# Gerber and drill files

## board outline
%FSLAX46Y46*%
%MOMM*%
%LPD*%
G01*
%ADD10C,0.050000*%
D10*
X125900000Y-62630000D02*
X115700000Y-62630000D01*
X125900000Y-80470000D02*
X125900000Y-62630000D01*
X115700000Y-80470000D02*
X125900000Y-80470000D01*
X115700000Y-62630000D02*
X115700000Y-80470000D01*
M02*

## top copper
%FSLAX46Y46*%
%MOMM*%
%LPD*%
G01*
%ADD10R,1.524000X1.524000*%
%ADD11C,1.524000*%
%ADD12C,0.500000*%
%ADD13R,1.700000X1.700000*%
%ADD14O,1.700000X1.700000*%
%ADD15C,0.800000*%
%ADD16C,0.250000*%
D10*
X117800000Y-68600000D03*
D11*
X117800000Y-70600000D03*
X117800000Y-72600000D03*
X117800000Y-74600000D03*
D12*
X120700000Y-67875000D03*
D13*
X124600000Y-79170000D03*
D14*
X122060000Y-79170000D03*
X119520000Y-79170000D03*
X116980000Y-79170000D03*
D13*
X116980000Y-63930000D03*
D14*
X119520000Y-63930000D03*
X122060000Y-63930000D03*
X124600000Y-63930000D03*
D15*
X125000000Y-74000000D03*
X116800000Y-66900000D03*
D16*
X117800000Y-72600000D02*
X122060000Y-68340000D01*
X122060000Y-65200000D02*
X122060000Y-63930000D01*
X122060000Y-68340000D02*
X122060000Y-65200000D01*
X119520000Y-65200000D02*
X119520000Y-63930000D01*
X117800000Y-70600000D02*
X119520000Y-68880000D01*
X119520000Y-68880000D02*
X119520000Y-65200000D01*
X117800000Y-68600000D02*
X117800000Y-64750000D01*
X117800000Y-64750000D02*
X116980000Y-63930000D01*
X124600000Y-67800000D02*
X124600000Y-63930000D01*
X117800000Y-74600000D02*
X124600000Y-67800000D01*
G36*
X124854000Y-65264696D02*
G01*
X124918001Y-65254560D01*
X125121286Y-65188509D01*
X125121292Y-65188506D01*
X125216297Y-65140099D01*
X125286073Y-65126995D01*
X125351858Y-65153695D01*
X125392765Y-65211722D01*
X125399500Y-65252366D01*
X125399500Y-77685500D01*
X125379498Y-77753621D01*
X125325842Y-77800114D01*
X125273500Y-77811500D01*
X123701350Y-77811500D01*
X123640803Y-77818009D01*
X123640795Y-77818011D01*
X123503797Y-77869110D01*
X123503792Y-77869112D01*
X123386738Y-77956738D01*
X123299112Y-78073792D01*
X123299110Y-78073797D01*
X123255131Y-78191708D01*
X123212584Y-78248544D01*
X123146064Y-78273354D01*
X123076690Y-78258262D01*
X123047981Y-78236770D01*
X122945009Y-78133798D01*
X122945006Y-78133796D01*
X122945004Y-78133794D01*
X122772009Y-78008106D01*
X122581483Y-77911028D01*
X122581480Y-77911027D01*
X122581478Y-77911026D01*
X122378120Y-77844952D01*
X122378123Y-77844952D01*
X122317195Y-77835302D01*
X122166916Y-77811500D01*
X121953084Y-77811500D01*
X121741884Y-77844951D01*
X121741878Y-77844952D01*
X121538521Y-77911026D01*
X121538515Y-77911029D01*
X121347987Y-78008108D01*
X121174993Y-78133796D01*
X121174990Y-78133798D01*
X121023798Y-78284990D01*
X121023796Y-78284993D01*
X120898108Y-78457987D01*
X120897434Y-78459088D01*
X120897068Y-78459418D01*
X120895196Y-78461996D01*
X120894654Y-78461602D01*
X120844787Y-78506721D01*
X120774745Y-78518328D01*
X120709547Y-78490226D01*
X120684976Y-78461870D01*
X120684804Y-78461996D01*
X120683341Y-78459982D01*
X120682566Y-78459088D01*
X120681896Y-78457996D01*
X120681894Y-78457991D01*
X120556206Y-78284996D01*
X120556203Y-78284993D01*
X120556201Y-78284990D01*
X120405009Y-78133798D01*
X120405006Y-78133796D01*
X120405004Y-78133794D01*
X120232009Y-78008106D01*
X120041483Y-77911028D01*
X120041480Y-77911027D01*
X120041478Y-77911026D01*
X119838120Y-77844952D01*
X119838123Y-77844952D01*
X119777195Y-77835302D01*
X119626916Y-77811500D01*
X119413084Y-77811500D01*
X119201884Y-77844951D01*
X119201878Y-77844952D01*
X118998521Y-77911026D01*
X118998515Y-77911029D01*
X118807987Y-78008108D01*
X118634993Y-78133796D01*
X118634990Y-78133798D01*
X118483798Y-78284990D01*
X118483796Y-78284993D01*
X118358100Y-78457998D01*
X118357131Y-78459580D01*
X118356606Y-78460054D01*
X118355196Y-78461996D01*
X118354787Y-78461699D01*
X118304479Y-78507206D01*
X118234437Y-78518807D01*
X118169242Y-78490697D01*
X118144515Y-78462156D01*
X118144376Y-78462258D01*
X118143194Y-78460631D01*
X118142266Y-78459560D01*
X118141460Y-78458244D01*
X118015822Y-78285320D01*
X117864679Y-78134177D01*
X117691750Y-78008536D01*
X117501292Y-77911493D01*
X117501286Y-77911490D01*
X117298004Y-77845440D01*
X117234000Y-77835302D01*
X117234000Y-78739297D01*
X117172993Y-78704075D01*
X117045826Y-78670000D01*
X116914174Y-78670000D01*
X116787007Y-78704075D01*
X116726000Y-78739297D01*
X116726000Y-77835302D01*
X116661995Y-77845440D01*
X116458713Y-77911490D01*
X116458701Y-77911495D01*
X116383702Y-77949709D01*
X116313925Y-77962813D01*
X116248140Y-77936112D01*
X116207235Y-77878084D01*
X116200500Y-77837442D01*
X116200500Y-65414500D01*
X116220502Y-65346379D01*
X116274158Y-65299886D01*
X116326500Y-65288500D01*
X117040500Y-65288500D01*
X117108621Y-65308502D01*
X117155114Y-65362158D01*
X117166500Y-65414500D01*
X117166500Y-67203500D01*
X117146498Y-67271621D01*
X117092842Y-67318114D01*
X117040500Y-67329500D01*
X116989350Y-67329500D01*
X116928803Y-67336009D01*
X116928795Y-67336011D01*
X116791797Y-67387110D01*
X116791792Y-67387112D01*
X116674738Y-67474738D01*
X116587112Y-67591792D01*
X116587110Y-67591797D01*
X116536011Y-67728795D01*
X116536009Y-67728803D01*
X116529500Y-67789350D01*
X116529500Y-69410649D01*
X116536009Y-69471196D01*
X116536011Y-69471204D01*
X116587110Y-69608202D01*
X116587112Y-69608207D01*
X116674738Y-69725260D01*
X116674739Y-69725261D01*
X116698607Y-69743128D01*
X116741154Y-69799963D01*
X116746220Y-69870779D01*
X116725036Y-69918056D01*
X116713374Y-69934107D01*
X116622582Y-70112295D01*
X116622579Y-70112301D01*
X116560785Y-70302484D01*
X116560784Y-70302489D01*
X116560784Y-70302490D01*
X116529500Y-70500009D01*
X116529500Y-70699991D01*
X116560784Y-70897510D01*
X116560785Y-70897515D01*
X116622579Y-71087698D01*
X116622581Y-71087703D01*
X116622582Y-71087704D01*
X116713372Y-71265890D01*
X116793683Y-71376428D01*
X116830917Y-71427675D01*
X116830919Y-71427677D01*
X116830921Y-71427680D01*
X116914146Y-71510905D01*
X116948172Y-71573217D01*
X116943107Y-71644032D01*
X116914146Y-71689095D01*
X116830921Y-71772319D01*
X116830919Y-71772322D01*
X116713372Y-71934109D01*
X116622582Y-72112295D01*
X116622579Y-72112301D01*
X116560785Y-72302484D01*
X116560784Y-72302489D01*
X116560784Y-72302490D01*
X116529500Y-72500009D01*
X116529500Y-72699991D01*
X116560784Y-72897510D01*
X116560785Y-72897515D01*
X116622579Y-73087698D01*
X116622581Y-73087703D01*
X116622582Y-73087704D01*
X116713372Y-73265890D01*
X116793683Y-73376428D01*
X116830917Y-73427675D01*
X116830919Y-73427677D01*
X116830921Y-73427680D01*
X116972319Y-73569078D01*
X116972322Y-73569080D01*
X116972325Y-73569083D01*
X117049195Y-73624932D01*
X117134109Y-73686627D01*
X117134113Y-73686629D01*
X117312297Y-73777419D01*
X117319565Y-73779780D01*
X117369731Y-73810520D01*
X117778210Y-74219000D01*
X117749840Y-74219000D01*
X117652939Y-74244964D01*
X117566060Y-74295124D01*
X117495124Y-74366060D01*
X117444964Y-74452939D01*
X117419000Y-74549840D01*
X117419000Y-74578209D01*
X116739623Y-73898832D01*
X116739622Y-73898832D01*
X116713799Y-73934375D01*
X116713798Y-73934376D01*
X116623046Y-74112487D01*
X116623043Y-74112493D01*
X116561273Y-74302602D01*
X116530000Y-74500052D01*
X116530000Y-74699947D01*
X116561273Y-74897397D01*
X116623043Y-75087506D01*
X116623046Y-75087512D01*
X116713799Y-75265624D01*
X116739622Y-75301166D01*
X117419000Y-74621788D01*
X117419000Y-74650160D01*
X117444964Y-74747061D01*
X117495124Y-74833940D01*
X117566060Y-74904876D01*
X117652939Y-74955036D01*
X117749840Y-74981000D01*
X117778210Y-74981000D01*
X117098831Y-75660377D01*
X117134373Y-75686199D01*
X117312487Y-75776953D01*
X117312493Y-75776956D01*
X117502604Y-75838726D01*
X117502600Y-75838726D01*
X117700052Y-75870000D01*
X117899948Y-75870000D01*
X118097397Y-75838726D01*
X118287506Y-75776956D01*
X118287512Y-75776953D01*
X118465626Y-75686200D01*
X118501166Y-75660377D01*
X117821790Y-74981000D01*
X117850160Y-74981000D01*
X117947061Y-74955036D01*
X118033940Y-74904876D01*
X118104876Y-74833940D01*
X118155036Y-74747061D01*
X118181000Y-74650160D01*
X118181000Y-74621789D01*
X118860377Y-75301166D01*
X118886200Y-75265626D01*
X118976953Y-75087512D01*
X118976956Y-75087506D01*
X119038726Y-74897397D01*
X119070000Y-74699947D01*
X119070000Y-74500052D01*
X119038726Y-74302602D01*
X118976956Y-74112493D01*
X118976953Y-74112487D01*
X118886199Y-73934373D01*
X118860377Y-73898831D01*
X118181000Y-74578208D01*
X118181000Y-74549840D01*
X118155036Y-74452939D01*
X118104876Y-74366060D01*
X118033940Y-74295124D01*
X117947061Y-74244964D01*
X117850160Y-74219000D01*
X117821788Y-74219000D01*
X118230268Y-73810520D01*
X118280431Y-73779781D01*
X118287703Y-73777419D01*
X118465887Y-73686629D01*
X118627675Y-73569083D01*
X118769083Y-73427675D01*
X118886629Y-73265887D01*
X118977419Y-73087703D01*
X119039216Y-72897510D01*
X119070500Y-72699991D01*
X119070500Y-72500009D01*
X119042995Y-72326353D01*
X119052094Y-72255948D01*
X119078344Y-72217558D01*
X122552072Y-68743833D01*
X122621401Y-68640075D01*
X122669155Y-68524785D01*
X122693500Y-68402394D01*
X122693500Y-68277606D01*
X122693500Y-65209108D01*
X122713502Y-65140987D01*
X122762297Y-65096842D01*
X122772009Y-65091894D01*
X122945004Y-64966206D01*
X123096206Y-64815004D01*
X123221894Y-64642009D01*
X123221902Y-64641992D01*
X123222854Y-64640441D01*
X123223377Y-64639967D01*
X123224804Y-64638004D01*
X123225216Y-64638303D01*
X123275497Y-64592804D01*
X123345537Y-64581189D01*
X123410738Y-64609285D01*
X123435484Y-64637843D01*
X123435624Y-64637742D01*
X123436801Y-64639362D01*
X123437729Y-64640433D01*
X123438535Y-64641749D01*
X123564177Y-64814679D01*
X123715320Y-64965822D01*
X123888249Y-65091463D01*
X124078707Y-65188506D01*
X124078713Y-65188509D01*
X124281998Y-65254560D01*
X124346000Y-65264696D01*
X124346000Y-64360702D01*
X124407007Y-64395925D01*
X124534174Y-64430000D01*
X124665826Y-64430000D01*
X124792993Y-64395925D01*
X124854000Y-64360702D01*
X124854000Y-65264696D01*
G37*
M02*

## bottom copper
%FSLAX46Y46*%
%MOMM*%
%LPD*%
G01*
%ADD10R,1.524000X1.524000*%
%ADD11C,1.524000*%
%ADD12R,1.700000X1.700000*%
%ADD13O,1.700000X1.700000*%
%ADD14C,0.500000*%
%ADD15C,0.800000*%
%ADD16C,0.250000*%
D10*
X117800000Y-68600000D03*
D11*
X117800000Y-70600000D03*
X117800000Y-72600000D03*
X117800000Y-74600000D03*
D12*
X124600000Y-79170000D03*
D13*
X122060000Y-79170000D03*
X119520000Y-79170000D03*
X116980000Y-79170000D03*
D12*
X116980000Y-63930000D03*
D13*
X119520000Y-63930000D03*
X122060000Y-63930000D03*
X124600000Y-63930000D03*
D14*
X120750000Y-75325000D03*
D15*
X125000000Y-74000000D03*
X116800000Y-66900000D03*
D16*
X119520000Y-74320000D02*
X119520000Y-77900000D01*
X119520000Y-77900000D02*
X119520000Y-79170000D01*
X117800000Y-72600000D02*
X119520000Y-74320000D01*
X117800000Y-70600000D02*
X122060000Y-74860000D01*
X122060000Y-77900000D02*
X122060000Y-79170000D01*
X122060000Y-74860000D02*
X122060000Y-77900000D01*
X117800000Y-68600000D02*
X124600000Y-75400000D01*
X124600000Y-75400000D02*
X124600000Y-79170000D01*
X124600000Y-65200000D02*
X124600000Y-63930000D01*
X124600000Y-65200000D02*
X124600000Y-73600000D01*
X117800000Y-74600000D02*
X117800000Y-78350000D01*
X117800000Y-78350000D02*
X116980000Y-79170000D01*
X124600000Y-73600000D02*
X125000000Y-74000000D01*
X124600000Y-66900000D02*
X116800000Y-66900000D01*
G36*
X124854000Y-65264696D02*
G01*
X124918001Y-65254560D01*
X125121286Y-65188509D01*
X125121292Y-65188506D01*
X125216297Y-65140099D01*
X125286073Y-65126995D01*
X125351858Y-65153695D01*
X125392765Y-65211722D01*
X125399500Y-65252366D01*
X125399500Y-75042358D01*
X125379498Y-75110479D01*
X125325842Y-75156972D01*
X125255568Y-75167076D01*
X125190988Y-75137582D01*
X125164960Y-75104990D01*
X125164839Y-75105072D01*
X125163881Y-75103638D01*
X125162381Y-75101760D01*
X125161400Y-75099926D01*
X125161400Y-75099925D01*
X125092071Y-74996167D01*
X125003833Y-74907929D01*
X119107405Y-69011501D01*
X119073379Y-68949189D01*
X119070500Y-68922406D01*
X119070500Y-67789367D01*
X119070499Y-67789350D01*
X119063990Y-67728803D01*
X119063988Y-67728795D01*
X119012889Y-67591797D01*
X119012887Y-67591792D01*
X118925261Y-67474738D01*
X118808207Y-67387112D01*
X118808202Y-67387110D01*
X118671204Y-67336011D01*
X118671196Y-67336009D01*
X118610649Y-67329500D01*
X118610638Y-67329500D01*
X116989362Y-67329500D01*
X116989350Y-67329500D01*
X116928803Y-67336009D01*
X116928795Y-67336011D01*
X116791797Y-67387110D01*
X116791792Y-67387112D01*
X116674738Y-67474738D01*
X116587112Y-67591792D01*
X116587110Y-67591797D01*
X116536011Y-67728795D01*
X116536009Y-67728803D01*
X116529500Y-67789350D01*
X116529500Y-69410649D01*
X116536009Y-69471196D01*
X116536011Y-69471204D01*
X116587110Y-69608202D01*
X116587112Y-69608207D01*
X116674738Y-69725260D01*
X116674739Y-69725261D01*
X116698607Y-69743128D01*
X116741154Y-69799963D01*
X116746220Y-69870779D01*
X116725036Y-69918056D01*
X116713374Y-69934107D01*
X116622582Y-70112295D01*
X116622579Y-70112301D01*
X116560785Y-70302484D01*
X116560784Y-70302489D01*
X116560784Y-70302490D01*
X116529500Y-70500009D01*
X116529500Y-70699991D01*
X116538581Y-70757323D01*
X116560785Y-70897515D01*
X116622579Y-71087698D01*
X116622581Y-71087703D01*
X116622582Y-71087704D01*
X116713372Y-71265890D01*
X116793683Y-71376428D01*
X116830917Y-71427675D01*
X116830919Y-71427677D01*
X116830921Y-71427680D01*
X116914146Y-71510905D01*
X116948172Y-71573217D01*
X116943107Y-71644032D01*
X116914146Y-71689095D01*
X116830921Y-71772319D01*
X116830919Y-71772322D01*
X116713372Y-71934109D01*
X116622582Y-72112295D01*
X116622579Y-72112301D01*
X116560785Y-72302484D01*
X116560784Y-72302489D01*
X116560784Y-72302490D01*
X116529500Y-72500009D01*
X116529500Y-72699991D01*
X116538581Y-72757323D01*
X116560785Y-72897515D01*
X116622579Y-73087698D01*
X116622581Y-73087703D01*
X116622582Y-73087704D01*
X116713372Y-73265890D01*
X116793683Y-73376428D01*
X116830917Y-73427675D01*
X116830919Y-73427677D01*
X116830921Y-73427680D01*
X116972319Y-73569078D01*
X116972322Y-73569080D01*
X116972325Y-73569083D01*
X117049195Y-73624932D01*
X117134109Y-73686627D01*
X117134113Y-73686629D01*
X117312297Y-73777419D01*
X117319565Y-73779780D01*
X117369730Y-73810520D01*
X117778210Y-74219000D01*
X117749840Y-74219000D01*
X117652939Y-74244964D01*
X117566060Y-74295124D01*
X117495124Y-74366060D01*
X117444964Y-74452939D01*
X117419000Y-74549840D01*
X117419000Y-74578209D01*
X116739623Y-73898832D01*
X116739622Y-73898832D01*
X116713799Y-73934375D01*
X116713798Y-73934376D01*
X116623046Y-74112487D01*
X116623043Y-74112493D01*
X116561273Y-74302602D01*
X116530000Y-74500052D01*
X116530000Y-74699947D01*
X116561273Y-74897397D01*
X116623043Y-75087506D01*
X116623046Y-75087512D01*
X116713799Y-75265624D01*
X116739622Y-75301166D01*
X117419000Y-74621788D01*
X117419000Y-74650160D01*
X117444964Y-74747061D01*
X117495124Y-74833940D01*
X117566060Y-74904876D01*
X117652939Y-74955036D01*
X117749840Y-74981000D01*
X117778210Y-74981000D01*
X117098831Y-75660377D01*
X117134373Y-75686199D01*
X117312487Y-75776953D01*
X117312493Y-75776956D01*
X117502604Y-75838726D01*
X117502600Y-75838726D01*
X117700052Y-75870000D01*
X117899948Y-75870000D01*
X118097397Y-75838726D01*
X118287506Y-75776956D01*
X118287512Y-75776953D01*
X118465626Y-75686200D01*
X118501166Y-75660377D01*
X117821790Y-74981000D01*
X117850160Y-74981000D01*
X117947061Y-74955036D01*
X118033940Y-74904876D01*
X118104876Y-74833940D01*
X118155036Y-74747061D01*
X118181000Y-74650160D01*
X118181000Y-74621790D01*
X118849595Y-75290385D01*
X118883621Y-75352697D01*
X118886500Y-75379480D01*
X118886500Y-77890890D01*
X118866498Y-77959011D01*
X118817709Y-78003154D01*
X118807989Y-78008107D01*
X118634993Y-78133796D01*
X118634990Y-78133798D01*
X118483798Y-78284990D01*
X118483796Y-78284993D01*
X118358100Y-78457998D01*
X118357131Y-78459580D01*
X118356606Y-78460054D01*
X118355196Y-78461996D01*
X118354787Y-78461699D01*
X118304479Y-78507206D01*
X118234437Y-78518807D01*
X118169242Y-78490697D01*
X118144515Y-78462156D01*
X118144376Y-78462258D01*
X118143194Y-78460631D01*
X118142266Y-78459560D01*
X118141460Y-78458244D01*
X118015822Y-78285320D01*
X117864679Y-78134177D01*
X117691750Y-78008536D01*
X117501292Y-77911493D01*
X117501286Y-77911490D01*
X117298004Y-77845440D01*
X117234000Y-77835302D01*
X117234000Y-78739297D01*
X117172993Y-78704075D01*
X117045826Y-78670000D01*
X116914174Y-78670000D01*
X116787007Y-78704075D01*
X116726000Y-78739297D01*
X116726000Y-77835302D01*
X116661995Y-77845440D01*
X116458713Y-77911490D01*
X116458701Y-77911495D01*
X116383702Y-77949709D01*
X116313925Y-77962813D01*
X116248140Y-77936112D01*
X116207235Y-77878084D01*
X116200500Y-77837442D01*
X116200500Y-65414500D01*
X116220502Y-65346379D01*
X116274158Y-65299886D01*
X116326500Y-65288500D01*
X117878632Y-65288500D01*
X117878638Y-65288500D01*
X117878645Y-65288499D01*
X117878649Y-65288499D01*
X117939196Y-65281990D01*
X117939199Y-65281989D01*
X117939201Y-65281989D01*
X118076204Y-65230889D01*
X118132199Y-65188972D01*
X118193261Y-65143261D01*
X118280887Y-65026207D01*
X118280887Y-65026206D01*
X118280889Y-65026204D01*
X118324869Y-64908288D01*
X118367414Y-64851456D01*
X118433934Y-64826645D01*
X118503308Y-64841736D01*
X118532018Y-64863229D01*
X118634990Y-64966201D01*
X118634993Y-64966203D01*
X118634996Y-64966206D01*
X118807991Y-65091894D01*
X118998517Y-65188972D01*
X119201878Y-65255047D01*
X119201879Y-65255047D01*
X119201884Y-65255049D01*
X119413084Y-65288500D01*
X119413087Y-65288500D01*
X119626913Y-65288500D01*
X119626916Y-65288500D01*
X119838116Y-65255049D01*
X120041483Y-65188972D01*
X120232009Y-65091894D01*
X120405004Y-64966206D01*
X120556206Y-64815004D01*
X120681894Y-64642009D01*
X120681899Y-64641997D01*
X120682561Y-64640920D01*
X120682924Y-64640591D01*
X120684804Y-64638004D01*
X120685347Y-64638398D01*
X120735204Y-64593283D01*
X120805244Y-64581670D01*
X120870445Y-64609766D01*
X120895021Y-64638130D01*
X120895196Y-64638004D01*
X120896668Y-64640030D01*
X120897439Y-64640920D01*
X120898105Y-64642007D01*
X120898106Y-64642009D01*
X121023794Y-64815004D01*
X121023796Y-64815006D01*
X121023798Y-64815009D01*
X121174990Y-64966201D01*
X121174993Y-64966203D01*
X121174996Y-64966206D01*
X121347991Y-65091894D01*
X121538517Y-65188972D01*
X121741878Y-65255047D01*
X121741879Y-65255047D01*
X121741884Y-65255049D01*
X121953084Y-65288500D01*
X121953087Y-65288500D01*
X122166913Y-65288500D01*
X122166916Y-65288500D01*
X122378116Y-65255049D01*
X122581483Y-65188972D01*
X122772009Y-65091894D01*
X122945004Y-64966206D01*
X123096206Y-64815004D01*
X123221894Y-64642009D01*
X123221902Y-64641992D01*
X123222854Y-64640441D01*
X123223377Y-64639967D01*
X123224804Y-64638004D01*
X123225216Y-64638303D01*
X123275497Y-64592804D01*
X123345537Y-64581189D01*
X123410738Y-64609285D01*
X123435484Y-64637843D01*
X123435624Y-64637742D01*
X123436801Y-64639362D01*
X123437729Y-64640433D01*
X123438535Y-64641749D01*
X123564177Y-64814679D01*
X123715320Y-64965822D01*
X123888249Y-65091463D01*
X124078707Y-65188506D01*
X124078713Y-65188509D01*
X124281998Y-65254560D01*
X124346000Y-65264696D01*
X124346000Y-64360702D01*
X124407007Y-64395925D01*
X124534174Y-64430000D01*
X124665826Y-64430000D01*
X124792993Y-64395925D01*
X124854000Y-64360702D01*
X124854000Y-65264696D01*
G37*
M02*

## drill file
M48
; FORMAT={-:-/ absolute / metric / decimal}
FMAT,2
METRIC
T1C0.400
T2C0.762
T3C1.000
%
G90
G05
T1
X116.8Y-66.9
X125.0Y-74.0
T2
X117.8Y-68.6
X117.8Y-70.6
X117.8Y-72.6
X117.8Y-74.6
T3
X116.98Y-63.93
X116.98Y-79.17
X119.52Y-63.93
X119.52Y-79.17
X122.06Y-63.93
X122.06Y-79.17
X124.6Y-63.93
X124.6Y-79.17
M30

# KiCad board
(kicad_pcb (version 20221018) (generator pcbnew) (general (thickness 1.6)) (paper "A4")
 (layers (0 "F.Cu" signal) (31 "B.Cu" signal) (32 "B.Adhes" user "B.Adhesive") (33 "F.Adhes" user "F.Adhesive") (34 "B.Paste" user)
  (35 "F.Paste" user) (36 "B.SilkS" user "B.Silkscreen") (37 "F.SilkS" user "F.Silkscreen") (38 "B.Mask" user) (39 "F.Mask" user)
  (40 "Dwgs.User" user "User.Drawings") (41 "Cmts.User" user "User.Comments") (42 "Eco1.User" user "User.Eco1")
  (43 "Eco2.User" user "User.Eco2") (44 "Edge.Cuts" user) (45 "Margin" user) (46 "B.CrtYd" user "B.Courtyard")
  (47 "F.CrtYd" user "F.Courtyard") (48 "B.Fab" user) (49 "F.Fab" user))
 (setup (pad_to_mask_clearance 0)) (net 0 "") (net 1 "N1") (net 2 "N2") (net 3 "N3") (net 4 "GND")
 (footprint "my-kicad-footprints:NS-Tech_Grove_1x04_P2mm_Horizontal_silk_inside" (layer "F.Cu") (at 117.8 71.6)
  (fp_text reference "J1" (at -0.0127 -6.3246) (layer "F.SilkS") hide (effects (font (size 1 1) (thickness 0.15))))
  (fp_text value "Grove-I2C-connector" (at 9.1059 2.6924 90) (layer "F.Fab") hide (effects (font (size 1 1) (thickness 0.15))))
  (pad "1" thru_hole rect (at 0 -3) (size 1.524 1.524) (drill 0.762) (layers "*.Cu" "*.Mask") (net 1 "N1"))
  (pad "2" thru_hole circle (at 0 -1) (size 1.524 1.524) (drill 0.762) (layers "*.Cu" "*.Mask") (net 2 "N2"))
  (pad "3" thru_hole circle (at 0 1) (size 1.524 1.524) (drill 0.762) (layers "*.Cu" "*.Mask") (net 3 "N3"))
  (pad "4" thru_hole circle (at 0 3) (size 1.524 1.524) (drill 0.762) (layers "*.Cu" "*.Mask") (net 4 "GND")))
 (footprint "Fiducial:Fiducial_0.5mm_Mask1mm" (layer "F.Cu") (at 120.7 67.875)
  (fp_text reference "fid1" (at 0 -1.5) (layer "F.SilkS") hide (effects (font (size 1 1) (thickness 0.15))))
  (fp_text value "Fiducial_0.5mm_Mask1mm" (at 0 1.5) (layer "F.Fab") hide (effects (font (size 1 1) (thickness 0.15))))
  (pad "" smd circle (at 0 0) (size 0.5 0.5) (layers "F.Cu" "F.Mask") (solder_mask_margin 0.25) (clearance 0.25)))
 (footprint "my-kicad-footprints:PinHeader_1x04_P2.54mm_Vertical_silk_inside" (layer "B.Cu") (at 124.6 79.17 90)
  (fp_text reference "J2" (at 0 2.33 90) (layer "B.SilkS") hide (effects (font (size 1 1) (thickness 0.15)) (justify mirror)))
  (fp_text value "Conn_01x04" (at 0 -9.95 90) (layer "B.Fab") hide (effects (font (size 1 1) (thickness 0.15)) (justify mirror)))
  (pad "1" thru_hole rect (at 0 0 90) (size 1.7 1.7) (drill 1) (layers "*.Cu" "*.Mask") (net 1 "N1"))
  (pad "2" thru_hole oval (at 0 -2.54 90) (size 1.7 1.7) (drill 1) (layers "*.Cu" "*.Mask") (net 2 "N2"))
  (pad "3" thru_hole oval (at 0 -5.08 90) (size 1.7 1.7) (drill 1) (layers "*.Cu" "*.Mask") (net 3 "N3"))
  (pad "4" thru_hole oval (at 0 -7.62 90) (size 1.7 1.7) (drill 1) (layers "*.Cu" "*.Mask") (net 4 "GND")))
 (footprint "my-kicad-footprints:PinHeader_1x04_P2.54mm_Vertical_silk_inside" (layer "B.Cu") (at 116.98 63.93 -90)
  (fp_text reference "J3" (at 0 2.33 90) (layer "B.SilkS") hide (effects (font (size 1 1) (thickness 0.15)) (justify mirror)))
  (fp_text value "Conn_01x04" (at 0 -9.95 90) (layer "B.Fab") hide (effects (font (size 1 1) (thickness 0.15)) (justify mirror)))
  (pad "1" thru_hole rect (at 0 0 270) (size 1.7 1.7) (drill 1) (layers "*.Cu" "*.Mask") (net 1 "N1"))
  (pad "2" thru_hole oval (at 0 -2.54 270) (size 1.7 1.7) (drill 1) (layers "*.Cu" "*.Mask") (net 2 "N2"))
  (pad "3" thru_hole oval (at 0 -5.08 270) (size 1.7 1.7) (drill 1) (layers "*.Cu" "*.Mask") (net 3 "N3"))
  (pad "4" thru_hole oval (at 0 -7.62 270) (size 1.7 1.7) (drill 1) (layers "*.Cu" "*.Mask") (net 4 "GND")))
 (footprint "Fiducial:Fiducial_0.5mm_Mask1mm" (layer "B.Cu") (at 120.75 75.325)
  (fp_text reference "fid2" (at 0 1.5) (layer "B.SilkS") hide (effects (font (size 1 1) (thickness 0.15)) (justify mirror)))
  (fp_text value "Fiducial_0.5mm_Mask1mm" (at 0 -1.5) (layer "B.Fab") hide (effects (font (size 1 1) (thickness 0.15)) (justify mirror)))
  (pad "" smd circle (at 0 0) (size 0.5 0.5) (layers "B.Cu" "B.Mask") (solder_mask_margin 0.25) (clearance 0.25)))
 (gr_line (start 125.9 62.63) (end 115.7 62.63) (stroke (width 0.05) (type solid)) (layer "Edge.Cuts"))
 (gr_line (start 125.9 80.47) (end 125.9 62.63) (stroke (width 0.05) (type solid)) (layer "Edge.Cuts"))
 (gr_line (start 115.7 80.47) (end 125.9 80.47) (stroke (width 0.05) (type solid)) (layer "Edge.Cuts"))
 (gr_line (start 115.7 62.63) (end 115.7 80.47) (stroke (width 0.05) (type solid)) (layer "Edge.Cuts"))
 (segment (start 117.8 72.6) (end 122.06 68.34) (width 0.25) (layer "F.Cu") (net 3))
 (segment (start 122.06 65.2) (end 122.06 63.93) (width 0.25) (layer "F.Cu") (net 3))
 (segment (start 122.06 68.34) (end 122.06 65.2) (width 0.25) (layer "F.Cu") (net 3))
 (segment (start 119.52 74.32) (end 119.52 77.9) (width 0.25) (layer "B.Cu") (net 3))
 (segment (start 119.52 77.9) (end 119.52 79.17) (width 0.25) (layer "B.Cu") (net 3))
 (segment (start 117.8 72.6) (end 119.52 74.32) (width 0.25) (layer "B.Cu") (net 3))
 (segment (start 119.52 65.2) (end 119.52 63.93) (width 0.25) (layer "F.Cu") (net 2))
 (segment (start 117.8 70.6) (end 119.52 68.88) (width 0.25) (layer "F.Cu") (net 2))
 (segment (start 119.52 68.88) (end 119.52 65.2) (width 0.25) (layer "F.Cu") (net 2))
 (segment (start 117.8 70.6) (end 122.06 74.86) (width 0.25) (layer "B.Cu") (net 2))
 (segment (start 122.06 77.9) (end 122.06 79.17) (width 0.25) (layer "B.Cu") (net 2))
 (segment (start 122.06 74.86) (end 122.06 77.9) (width 0.25) (layer "B.Cu") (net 2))
 (segment (start 117.8 68.6) (end 117.8 64.75) (width 0.25) (layer "F.Cu") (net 1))
 (segment (start 117.8 64.75) (end 116.98 63.93) (width 0.25) (layer "F.Cu") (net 1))
 (segment (start 117.8 68.6) (end 124.6 75.4) (width 0.25) (layer "B.Cu") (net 1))
 (segment (start 124.6 75.4) (end 124.6 79.17) (width 0.25) (layer "B.Cu") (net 1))
 (segment (start 124.6 67.8) (end 124.6 63.93) (width 0.25) (layer "F.Cu") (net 4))
 (segment (start 117.8 74.6) (end 124.6 67.8) (width 0.25) (layer "F.Cu") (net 4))
 (via (at 125 74) (size 0.8) (drill 0.4) (layers "F.Cu" "B.Cu") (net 4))
 (via (at 116.8 66.9) (size 0.8) (drill 0.4) (layers "F.Cu" "B.Cu") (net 4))
 (segment (start 124.6 65.2) (end 124.6 63.93) (width 0.25) (layer "B.Cu") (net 4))
 (segment (start 124.6 65.2) (end 124.6 73.6) (width 0.25) (layer "B.Cu") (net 4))
 (segment (start 117.8 74.6) (end 117.8 78.35) (width 0.25) (layer "B.Cu") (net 4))
 (segment (start 117.8 78.35) (end 116.98 79.17) (width 0.25) (layer "B.Cu") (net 4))
 (segment (start 124.6 73.6) (end 125 74) (width 0.25) (layer "B.Cu") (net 4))
 (segment (start 124.6 66.9) (end 116.8 66.9) (width 0.25) (layer "B.Cu") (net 4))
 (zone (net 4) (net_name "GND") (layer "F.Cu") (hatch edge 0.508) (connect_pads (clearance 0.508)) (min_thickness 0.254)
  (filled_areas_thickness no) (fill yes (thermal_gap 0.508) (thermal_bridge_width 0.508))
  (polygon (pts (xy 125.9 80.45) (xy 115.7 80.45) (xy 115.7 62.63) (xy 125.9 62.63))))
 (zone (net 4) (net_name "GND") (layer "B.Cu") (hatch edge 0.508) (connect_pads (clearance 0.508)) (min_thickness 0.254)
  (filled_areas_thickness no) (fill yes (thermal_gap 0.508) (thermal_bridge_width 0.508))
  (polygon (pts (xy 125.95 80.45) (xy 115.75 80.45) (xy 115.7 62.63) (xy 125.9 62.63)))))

